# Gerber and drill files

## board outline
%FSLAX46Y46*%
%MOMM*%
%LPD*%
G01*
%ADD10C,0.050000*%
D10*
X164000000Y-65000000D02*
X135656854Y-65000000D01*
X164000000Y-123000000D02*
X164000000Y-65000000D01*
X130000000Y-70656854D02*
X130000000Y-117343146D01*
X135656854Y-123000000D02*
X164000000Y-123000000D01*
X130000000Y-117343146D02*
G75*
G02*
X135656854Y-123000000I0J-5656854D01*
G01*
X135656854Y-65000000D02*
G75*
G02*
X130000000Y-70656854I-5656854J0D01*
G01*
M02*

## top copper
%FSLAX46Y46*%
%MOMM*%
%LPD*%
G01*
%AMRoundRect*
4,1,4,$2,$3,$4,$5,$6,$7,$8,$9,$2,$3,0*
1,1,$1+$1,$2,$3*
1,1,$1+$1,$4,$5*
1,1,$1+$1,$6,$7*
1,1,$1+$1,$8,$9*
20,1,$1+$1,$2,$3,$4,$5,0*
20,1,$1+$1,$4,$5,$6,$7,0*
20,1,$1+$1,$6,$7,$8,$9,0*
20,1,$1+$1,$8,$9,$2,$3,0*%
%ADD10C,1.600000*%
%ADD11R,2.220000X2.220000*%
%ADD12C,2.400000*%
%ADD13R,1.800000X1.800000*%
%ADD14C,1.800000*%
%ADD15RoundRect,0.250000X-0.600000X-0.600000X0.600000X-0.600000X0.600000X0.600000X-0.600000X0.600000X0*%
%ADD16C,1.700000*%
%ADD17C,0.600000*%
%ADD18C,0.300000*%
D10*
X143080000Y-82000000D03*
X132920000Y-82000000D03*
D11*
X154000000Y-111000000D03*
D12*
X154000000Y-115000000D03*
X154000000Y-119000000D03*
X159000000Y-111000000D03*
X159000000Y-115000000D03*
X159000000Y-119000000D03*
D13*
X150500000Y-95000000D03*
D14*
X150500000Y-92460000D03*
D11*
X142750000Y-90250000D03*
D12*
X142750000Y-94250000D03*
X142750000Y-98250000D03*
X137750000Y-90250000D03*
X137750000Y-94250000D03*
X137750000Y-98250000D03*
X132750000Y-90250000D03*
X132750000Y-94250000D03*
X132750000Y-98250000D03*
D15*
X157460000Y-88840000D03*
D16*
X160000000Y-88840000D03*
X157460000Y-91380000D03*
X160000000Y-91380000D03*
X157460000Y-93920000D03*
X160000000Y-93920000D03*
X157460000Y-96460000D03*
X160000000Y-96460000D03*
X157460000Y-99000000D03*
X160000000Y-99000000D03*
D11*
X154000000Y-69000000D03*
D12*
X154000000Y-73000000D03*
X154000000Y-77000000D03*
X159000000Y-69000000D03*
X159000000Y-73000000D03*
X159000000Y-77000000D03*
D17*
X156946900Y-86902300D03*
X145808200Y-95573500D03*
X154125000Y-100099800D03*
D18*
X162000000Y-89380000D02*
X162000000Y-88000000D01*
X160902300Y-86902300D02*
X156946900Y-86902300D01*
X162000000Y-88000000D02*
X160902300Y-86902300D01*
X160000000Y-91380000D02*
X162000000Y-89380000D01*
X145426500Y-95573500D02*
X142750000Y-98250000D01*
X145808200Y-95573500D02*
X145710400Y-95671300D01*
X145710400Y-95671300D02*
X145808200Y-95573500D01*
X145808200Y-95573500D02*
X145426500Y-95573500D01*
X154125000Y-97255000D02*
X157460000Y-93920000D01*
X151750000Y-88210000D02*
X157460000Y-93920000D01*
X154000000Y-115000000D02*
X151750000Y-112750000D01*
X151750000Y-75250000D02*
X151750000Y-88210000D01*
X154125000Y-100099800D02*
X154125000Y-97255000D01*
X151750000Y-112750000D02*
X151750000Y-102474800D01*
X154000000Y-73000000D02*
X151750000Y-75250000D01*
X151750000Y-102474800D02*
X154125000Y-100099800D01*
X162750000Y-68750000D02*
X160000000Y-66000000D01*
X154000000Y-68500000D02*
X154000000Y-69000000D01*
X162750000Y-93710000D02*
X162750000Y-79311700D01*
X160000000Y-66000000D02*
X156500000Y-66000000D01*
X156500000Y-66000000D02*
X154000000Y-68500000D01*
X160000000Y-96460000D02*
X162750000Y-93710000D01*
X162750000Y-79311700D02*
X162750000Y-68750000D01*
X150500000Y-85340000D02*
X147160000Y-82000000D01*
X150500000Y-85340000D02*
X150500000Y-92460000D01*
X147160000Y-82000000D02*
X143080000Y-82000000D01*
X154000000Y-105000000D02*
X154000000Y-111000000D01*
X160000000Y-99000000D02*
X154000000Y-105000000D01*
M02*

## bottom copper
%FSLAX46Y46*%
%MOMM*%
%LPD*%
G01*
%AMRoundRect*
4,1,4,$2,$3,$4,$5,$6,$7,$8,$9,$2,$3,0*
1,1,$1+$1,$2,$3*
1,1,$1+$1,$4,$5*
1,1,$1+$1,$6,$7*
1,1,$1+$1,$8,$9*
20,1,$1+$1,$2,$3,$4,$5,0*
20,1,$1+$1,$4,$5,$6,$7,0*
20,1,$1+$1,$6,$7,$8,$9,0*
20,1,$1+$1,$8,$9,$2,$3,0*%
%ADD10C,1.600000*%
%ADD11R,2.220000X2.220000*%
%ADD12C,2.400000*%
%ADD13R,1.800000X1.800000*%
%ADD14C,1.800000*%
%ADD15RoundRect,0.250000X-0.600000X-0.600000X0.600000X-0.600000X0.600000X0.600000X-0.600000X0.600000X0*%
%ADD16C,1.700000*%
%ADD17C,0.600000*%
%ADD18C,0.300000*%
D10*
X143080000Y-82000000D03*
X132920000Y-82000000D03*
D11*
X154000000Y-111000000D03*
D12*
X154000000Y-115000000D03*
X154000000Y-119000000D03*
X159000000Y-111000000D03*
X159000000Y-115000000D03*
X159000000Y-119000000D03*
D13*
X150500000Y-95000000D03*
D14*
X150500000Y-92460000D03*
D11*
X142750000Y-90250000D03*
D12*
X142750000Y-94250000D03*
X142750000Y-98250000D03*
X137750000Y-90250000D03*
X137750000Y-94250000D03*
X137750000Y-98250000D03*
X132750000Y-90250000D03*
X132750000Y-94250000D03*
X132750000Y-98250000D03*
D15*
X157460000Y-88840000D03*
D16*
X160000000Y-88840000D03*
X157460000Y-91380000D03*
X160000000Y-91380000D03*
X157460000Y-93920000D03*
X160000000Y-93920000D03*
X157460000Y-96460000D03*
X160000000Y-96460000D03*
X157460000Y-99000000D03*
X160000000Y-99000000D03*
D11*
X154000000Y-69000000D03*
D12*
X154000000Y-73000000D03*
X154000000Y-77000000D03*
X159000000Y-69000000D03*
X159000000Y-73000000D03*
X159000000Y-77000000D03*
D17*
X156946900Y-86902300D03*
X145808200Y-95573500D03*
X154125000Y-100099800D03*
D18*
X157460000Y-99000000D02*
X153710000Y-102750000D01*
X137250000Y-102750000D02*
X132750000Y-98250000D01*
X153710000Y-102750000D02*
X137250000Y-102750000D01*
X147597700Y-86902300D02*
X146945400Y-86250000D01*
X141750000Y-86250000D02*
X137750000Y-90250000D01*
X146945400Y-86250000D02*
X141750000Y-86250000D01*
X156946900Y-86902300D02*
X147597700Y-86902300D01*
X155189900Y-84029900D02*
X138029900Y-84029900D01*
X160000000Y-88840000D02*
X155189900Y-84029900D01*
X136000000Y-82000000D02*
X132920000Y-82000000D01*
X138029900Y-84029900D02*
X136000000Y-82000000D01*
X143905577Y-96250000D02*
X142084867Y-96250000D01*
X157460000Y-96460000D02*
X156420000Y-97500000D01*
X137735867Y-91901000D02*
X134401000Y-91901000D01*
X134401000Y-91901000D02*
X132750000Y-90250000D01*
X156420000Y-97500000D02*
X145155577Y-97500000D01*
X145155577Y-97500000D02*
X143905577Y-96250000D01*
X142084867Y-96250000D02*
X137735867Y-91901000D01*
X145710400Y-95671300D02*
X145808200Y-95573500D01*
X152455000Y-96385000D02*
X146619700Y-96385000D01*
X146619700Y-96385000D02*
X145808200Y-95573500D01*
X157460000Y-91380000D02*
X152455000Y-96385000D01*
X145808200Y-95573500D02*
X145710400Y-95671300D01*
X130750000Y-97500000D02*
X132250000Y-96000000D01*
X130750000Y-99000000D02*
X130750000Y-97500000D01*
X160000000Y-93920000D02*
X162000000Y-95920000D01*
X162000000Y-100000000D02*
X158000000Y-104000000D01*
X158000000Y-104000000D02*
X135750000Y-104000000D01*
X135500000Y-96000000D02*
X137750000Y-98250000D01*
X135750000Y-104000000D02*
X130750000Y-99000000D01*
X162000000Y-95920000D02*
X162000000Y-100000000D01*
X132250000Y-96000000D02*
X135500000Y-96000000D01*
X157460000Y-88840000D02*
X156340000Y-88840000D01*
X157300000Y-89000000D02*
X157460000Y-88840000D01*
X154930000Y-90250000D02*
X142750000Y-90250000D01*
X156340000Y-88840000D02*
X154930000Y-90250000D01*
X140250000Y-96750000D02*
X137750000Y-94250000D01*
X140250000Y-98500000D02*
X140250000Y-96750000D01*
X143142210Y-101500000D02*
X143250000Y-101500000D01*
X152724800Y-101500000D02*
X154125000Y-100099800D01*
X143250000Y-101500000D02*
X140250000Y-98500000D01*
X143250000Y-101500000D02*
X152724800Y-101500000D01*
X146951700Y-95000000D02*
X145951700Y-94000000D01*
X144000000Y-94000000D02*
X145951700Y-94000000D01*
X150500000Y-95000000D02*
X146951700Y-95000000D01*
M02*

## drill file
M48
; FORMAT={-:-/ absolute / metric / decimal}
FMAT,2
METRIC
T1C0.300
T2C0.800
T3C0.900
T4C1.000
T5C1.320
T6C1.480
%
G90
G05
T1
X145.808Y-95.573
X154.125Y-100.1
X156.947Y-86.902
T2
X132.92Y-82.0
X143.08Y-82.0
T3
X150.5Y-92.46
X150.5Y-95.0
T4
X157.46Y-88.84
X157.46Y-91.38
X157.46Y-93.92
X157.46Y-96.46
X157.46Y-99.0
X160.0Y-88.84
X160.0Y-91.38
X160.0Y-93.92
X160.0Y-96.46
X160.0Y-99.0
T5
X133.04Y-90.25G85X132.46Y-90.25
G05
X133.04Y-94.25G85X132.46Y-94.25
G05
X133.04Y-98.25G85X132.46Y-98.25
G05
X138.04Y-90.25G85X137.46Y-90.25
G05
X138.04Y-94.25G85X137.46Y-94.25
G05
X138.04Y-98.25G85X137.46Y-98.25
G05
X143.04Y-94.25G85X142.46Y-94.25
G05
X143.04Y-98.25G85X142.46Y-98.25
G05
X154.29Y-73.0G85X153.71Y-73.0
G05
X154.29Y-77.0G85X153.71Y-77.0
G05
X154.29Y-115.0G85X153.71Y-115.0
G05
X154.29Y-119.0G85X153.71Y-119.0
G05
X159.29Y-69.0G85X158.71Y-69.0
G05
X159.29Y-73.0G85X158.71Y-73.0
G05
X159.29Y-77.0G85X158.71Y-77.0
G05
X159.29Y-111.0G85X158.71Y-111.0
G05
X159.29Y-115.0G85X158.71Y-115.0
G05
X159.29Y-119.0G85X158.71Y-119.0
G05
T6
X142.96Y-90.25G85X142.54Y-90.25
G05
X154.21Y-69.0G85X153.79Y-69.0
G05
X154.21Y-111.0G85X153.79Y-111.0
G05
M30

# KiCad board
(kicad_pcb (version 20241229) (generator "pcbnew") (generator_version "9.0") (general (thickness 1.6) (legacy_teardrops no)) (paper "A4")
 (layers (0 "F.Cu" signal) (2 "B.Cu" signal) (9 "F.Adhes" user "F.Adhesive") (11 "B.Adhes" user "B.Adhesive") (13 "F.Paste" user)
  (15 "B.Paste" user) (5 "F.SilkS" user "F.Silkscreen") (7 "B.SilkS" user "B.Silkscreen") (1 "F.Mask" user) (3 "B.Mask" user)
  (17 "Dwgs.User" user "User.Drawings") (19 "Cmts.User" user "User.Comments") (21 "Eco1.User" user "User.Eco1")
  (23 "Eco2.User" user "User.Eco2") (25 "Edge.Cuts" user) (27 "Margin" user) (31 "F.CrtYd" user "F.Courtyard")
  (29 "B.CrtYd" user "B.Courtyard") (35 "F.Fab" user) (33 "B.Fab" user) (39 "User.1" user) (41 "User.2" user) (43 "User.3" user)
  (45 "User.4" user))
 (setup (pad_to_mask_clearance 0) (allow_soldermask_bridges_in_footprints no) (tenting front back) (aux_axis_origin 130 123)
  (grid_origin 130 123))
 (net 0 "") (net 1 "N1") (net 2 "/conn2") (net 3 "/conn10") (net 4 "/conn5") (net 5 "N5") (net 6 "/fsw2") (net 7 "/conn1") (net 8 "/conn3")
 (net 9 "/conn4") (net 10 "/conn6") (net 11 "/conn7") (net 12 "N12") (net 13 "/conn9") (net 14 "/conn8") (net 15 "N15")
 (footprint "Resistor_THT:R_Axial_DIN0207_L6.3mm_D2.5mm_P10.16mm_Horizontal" (layer "F.Cu") (at 143.08 82 180)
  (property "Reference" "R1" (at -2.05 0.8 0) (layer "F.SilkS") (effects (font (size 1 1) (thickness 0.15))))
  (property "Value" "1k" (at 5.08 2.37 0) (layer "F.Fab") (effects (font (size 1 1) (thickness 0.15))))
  (pad "1" thru_hole circle (at 0 0 180) (size 1.6 1.6) (drill 0.8) (layers "*.Cu" "*.Mask") (remove_unused_layers no) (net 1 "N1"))
  (pad "2" thru_hole circle (at 10.16 0 180) (size 1.6 1.6) (drill 0.8) (layers "*.Cu" "*.Mask") (remove_unused_layers no) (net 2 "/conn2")))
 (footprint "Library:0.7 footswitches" (layer "F.Cu") (at 154 111 -90)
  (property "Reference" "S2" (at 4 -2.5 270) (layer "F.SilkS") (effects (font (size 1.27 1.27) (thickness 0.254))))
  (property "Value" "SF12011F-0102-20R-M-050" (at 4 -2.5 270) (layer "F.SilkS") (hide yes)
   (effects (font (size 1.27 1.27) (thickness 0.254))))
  (pad "1" thru_hole rect (at 0 0 270) (size 2.22 2.22) (drill oval 1.48 1.9) (layers "*.Cu" "*.Mask") (remove_unused_layers no)
   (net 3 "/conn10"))
  (pad "2" thru_hole circle (at 4 0 270) (size 2.4 2.4) (drill oval 1.32 1.9) (layers "*.Cu" "*.Mask") (remove_unused_layers no)
   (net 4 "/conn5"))
  (pad "3" thru_hole circle (at 8 0 270) (size 2.4 2.4) (drill oval 1.32 1.9) (layers "*.Cu" "*.Mask") (remove_unused_layers no)
   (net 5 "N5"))
  (pad "4" thru_hole circle (at 0 -5 270) (size 2.4 2.4) (drill oval 1.32 1.9) (layers "*.Cu" "*.Mask") (remove_unused_layers no))
  (pad "5" thru_hole circle (at 4 -5 270) (size 2.4 2.4) (drill oval 1.32 1.9) (layers "*.Cu" "*.Mask") (remove_unused_layers no))
  (pad "6" thru_hole circle (at 8 -5 270) (size 2.4 2.4) (drill oval 1.32 1.9) (layers "*.Cu" "*.Mask") (remove_unused_layers no)))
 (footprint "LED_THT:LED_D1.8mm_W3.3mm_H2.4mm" (layer "F.Cu") (at 150.5 95 90)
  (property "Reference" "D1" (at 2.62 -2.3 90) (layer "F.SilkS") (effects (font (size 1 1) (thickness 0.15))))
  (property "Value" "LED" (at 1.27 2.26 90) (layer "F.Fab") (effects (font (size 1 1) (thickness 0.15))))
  (pad "1" thru_hole rect (at 0 0 90) (size 1.8 1.8) (drill 0.9) (layers "*.Cu" "*.Mask") (remove_unused_layers no) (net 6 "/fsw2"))
  (pad "2" thru_hole circle (at 2.54 0 90) (size 1.8 1.8) (drill 0.9) (layers "*.Cu" "*.Mask") (remove_unused_layers no) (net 1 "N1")))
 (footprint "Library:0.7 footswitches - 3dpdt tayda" (layer "F.Cu") (at 135.25 90.25 -90)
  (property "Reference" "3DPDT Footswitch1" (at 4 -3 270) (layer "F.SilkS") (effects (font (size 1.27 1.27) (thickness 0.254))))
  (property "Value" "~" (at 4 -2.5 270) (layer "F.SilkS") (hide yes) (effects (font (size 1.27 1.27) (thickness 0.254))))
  (pad "1" thru_hole rect (at 0 -7.5 270) (size 2.22 2.22) (drill oval 1.48 1.9) (layers "*.Cu" "*.Mask") (remove_unused_layers no)
   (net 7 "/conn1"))
  (pad "2" thru_hole circle (at 4 -7.5 270) (size 2.4 2.4) (drill oval 1.32 1.9) (layers "*.Cu" "*.Mask") (remove_unused_layers no)
   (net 6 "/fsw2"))
  (pad "3" thru_hole circle (at 8 -7.5 270) (size 2.4 2.4) (drill oval 1.32 1.9) (layers "*.Cu" "*.Mask") (remove_unused_layers no)
   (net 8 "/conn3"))
  (pad "4" thru_hole circle (at 0 -2.5 270) (size 2.4 2.4) (drill oval 1.32 1.9) (layers "*.Cu" "*.Mask") (remove_unused_layers no)
   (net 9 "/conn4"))
  (pad "5" thru_hole circle (at 4 -2.5 270) (size 2.4 2.4) (drill oval 1.32 1.9) (layers "*.Cu" "*.Mask") (remove_unused_layers no)
   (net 4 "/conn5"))
  (pad "6" thru_hole circle (at 8 -2.5 270) (size 2.4 2.4) (drill oval 1.32 1.9) (layers "*.Cu" "*.Mask") (remove_unused_layers no)
   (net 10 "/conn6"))
  (pad "7" thru_hole circle (at 0 2.5 270) (size 2.4 2.4) (drill oval 1.32 1.9) (layers "*.Cu" "*.Mask") (remove_unused_layers no)
   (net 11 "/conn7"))
  (pad "8" thru_hole circle (at 4 2.5 270) (size 2.4 2.4) (drill oval 1.32 1.9) (layers "*.Cu" "*.Mask") (remove_unused_layers no)
   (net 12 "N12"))
  (pad "9" thru_hole circle (at 8 2.5 270) (size 2.4 2.4) (drill oval 1.32 1.9) (layers "*.Cu" "*.Mask") (remove_unused_layers no)
   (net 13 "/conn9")))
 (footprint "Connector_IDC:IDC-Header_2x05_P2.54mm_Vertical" (layer "F.Cu") (at 157.46 88.84)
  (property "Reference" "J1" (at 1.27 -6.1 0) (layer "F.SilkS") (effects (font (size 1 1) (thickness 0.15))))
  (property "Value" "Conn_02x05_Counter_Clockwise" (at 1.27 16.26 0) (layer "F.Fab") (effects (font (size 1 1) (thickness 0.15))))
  (pad "1" thru_hole roundrect (at 0 0) (size 1.7 1.7) (drill 1) (layers "*.Cu" "*.Mask") (remove_unused_layers no)
   (roundrect_rratio 0.147059) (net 7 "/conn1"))
  (pad "2" thru_hole circle (at 2.54 0) (size 1.7 1.7) (drill 1) (layers "*.Cu" "*.Mask") (remove_unused_layers no) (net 2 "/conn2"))
  (pad "3" thru_hole circle (at 0 2.54) (size 1.7 1.7) (drill 1) (layers "*.Cu" "*.Mask") (remove_unused_layers no) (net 8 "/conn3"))
  (pad "4" thru_hole circle (at 2.54 2.54) (size 1.7 1.7) (drill 1) (layers "*.Cu" "*.Mask") (remove_unused_layers no) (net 9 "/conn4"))
  (pad "5" thru_hole circle (at 0 5.08) (size 1.7 1.7) (drill 1) (layers "*.Cu" "*.Mask") (remove_unused_layers no) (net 4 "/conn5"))
  (pad "6" thru_hole circle (at 2.54 5.08) (size 1.7 1.7) (drill 1) (layers "*.Cu" "*.Mask") (remove_unused_layers no) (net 10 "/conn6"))
  (pad "7" thru_hole circle (at 0 7.62) (size 1.7 1.7) (drill 1) (layers "*.Cu" "*.Mask") (remove_unused_layers no) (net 11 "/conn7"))
  (pad "8" thru_hole circle (at 2.54 7.62) (size 1.7 1.7) (drill 1) (layers "*.Cu" "*.Mask") (remove_unused_layers no) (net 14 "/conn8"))
  (pad "9" thru_hole circle (at 0 10.16) (size 1.7 1.7) (drill 1) (layers "*.Cu" "*.Mask") (remove_unused_layers no) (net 13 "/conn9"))
  (pad "10" thru_hole circle (at 2.54 10.16) (size 1.7 1.7) (drill 1) (layers "*.Cu" "*.Mask") (remove_unused_layers no) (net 3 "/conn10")))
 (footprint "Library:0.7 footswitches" (layer "F.Cu") (at 154 69 -90)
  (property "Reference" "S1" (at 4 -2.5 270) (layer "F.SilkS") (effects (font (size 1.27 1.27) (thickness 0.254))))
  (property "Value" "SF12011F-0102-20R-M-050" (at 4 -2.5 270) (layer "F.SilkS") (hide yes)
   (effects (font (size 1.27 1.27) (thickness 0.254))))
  (pad "1" thru_hole rect (at 0 0 270) (size 2.22 2.22) (drill oval 1.48 1.9) (layers "*.Cu" "*.Mask") (remove_unused_layers no)
   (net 14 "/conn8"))
  (pad "2" thru_hole circle (at 4 0 270) (size 2.4 2.4) (drill oval 1.32 1.9) (layers "*.Cu" "*.Mask") (remove_unused_layers no)
   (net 4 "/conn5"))
  (pad "3" thru_hole circle (at 8 0 270) (size 2.4 2.4) (drill oval 1.32 1.9) (layers "*.Cu" "*.Mask") (remove_unused_layers no)
   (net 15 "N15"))
  (pad "4" thru_hole circle (at 0 -5 270) (size 2.4 2.4) (drill oval 1.32 1.9) (layers "*.Cu" "*.Mask") (remove_unused_layers no))
  (pad "5" thru_hole circle (at 4 -5 270) (size 2.4 2.4) (drill oval 1.32 1.9) (layers "*.Cu" "*.Mask") (remove_unused_layers no))
  (pad "6" thru_hole circle (at 8 -5 270) (size 2.4 2.4) (drill oval 1.32 1.9) (layers "*.Cu" "*.Mask") (remove_unused_layers no)))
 (gr_line (start 164 65) (end 135.656854 65) (stroke (width 0.05) (type default)) (layer "Edge.Cuts"))
 (gr_line (start 164 123) (end 164 65) (stroke (width 0.05) (type default)) (layer "Edge.Cuts"))
 (gr_line (start 130 70.656854) (end 130 117.343146) (stroke (width 0.05) (type default)) (layer "Edge.Cuts"))
 (gr_line (start 135.656854 123) (end 164 123) (stroke (width 0.05) (type default)) (layer "Edge.Cuts"))
 (gr_arc (start 130 117.343146) (mid 134 119) (end 135.656854 123) (stroke (width 0.05) (type default)) (layer "Edge.Cuts"))
 (gr_arc (start 135.656854 65) (mid 134 69) (end 130 70.656854) (stroke (width 0.05) (type default)) (layer "Edge.Cuts"))
 (segment (start 157.46 99) (end 153.71 102.75) (width 0.3) (layer "B.Cu") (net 13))
 (segment (start 137.25 102.75) (end 132.75 98.25) (width 0.3) (layer "B.Cu") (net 13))
 (segment (start 153.71 102.75) (end 137.25 102.75) (width 0.3) (layer "B.Cu") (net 13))
 (segment (start 162 89.38) (end 162 88) (width 0.3) (layer "F.Cu") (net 9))
 (segment (start 160.9023 86.9023) (end 156.9469 86.9023) (width 0.3) (layer "F.Cu") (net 9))
 (segment (start 162 88) (end 160.9023 86.9023) (width 0.3) (layer "F.Cu") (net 9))
 (segment (start 160 91.38) (end 162 89.38) (width 0.3) (layer "F.Cu") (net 9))
 (via (at 156.9469 86.9023) (size 0.6) (drill 0.3) (layers "F.Cu" "B.Cu") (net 9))
 (segment (start 147.5977 86.9023) (end 146.9454 86.25) (width 0.3) (layer "B.Cu") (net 9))
 (segment (start 141.75 86.25) (end 137.75 90.25) (width 0.3) (layer "B.Cu") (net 9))
 (segment (start 146.9454 86.25) (end 141.75 86.25) (width 0.3) (layer "B.Cu") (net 9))
 (segment (start 156.9469 86.9023) (end 147.5977 86.9023) (width 0.3) (layer "B.Cu") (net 9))
 (segment (start 155.1899 84.0299) (end 138.0299 84.0299) (width 0.3) (layer "B.Cu") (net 2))
 (segment (start 160 88.84) (end 155.1899 84.0299) (width 0.3) (layer "B.Cu") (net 2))
 (segment (start 136 82) (end 132.92 82) (width 0.3) (layer "B.Cu") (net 2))
 (segment (start 138.0299 84.0299) (end 136 82) (width 0.3) (layer "B.Cu") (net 2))
 (segment (start 143.905577 96.25) (end 142.084867 96.25) (width 0.3) (layer "B.Cu") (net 11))
 (segment (start 157.46 96.46) (end 156.42 97.5) (width 0.3) (layer "B.Cu") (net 11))
 (segment (start 137.735867 91.901) (end 134.401 91.901) (width 0.3) (layer "B.Cu") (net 11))
 (segment (start 134.401 91.901) (end 132.75 90.25) (width 0.3) (layer "B.Cu") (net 11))
 (segment (start 156.42 97.5) (end 145.155577 97.5) (width 0.3) (layer "B.Cu") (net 11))
 (segment (start 145.155577 97.5) (end 143.905577 96.25) (width 0.3) (layer "B.Cu") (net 11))
 (segment (start 142.084867 96.25) (end 137.735867 91.901) (width 0.3) (layer "B.Cu") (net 11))
 (segment (start 145.4265 95.5735) (end 142.75 98.25) (width 0.3) (layer "F.Cu") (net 8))
 (segment (start 145.8082 95.5735) (end 145.7104 95.6713) (width 0.3) (layer "F.Cu") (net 8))
 (segment (start 145.7104 95.6713) (end 145.8082 95.5735) (width 0.3) (layer "F.Cu") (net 8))
 (segment (start 145.8082 95.5735) (end 145.4265 95.5735) (width 0.3) (layer "F.Cu") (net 8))
 (via (at 145.8082 95.5735) (size 0.6) (drill 0.3) (layers "F.Cu" "B.Cu") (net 8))
 (segment (start 145.7104 95.6713) (end 145.8082 95.5735) (width 0.3) (layer "B.Cu") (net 8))
 (segment (start 152.455 96.385) (end 146.6197 96.385) (width 0.3) (layer "B.Cu") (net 8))
 (segment (start 146.6197 96.385) (end 145.8082 95.5735) (width 0.3) (layer "B.Cu") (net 8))
 (segment (start 157.46 91.38) (end 152.455 96.385) (width 0.3) (layer "B.Cu") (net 8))
 (segment (start 145.8082 95.5735) (end 145.7104 95.6713) (width 0.3) (layer "B.Cu") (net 8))
 (segment (start 130.75 97.5) (end 132.25 96) (width 0.3) (layer "B.Cu") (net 10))
 (segment (start 130.75 99) (end 130.75 97.5) (width 0.3) (layer "B.Cu") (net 10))
 (segment (start 160 93.92) (end 162 95.92) (width 0.3) (layer "B.Cu") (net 10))
 (segment (start 162 100) (end 158 104) (width 0.3) (layer "B.Cu") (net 10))
 (segment (start 158 104) (end 135.75 104) (width 0.3) (layer "B.Cu") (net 10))
 (segment (start 135.5 96) (end 137.75 98.25) (width 0.3) (layer "B.Cu") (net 10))
 (segment (start 135.75 104) (end 130.75 99) (width 0.3) (layer "B.Cu") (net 10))
 (segment (start 162 95.92) (end 162 100) (width 0.3) (layer "B.Cu") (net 10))
 (segment (start 132.25 96) (end 135.5 96) (width 0.3) (layer "B.Cu") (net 10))
 (segment (start 157.46 88.84) (end 156.34 88.84) (width 0.3) (layer "B.Cu") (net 7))
 (segment (start 157.3 89) (end 157.46 88.84) (width 0.3) (layer "B.Cu") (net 7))
 (segment (start 154.93 90.25) (end 142.75 90.25) (width 0.3) (layer "B.Cu") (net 7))
 (segment (start 156.34 88.84) (end 154.93 90.25) (width 0.3) (layer "B.Cu") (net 7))
 (segment (start 154.125 97.255) (end 157.46 93.92) (width 0.3) (layer "F.Cu") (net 4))
 (segment (start 151.75 88.21) (end 157.46 93.92) (width 0.3) (layer "F.Cu") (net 4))
 (segment (start 154 115) (end 151.75 112.75) (width 0.3) (layer "F.Cu") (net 4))
 (segment (start 151.75 75.25) (end 151.75 88.21) (width 0.3) (layer "F.Cu") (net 4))
 (segment (start 154.125 100.0998) (end 154.125 97.255) (width 0.3) (layer "F.Cu") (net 4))
 (segment (start 151.75 112.75) (end 151.75 102.4748) (width 0.3) (layer "F.Cu") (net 4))
 (segment (start 154 73) (end 151.75 75.25) (width 0.3) (layer "F.Cu") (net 4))
 (segment (start 151.75 102.4748) (end 154.125 100.0998) (width 0.3) (layer "F.Cu") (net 4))
 (via (at 154.125 100.0998) (size 0.6) (drill 0.3) (layers "F.Cu" "B.Cu") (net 4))
 (segment (start 140.25 96.75) (end 137.75 94.25) (width 0.3) (layer "B.Cu") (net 4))
 (segment (start 140.25 98.5) (end 140.25 96.75) (width 0.3) (layer "B.Cu") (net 4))
 (segment (start 143.14221 101.5) (end 143.25 101.5) (width 0.3) (layer "B.Cu") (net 4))
 (segment (start 152.7248 101.5) (end 154.125 100.0998) (width 0.3) (layer "B.Cu") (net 4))
 (segment (start 143.25 101.5) (end 140.25 98.5) (width 0.3) (layer "B.Cu") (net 4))
 (segment (start 143.25 101.5) (end 152.7248 101.5) (width 0.3) (layer "B.Cu") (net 4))
 (segment (start 162.75 68.75) (end 160 66) (width 0.3) (layer "F.Cu") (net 14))
 (segment (start 154 68.5) (end 154 69) (width 0.3) (layer "F.Cu") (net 14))
 (segment (start 162.75 93.71) (end 162.75 79.3117) (width 0.3) (layer "F.Cu") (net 14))
 (segment (start 160 66) (end 156.5 66) (width 0.3) (layer "F.Cu") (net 14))
 (segment (start 156.5 66) (end 154 68.5) (width 0.3) (layer "F.Cu") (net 14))
 (segment (start 160 96.46) (end 162.75 93.71) (width 0.3) (layer "F.Cu") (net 14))
 (segment (start 162.75 79.3117) (end 162.75 68.75) (width 0.3) (layer "F.Cu") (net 14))
 (segment (start 150.5 85.34) (end 147.16 82) (width 0.3) (layer "F.Cu") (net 1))
 (segment (start 150.5 85.34) (end 150.5 92.46) (width 0.3) (layer "F.Cu") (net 1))
 (segment (start 147.16 82) (end 143.08 82) (width 0.3) (layer "F.Cu") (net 1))
 (segment (start 146.9517 95) (end 145.9517 94) (width 0.3) (layer "B.Cu") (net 6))
 (segment (start 144 94) (end 145.9517 94) (width 0.3) (layer "B.Cu") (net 6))
 (segment (start 150.5 95) (end 146.9517 95) (width 0.3) (layer "B.Cu") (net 6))
 (segment (start 154 105) (end 154 111) (width 0.3) (layer "F.Cu") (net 3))
 (segment (start 160 99) (end 154 105) (width 0.3) (layer "F.Cu") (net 3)))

